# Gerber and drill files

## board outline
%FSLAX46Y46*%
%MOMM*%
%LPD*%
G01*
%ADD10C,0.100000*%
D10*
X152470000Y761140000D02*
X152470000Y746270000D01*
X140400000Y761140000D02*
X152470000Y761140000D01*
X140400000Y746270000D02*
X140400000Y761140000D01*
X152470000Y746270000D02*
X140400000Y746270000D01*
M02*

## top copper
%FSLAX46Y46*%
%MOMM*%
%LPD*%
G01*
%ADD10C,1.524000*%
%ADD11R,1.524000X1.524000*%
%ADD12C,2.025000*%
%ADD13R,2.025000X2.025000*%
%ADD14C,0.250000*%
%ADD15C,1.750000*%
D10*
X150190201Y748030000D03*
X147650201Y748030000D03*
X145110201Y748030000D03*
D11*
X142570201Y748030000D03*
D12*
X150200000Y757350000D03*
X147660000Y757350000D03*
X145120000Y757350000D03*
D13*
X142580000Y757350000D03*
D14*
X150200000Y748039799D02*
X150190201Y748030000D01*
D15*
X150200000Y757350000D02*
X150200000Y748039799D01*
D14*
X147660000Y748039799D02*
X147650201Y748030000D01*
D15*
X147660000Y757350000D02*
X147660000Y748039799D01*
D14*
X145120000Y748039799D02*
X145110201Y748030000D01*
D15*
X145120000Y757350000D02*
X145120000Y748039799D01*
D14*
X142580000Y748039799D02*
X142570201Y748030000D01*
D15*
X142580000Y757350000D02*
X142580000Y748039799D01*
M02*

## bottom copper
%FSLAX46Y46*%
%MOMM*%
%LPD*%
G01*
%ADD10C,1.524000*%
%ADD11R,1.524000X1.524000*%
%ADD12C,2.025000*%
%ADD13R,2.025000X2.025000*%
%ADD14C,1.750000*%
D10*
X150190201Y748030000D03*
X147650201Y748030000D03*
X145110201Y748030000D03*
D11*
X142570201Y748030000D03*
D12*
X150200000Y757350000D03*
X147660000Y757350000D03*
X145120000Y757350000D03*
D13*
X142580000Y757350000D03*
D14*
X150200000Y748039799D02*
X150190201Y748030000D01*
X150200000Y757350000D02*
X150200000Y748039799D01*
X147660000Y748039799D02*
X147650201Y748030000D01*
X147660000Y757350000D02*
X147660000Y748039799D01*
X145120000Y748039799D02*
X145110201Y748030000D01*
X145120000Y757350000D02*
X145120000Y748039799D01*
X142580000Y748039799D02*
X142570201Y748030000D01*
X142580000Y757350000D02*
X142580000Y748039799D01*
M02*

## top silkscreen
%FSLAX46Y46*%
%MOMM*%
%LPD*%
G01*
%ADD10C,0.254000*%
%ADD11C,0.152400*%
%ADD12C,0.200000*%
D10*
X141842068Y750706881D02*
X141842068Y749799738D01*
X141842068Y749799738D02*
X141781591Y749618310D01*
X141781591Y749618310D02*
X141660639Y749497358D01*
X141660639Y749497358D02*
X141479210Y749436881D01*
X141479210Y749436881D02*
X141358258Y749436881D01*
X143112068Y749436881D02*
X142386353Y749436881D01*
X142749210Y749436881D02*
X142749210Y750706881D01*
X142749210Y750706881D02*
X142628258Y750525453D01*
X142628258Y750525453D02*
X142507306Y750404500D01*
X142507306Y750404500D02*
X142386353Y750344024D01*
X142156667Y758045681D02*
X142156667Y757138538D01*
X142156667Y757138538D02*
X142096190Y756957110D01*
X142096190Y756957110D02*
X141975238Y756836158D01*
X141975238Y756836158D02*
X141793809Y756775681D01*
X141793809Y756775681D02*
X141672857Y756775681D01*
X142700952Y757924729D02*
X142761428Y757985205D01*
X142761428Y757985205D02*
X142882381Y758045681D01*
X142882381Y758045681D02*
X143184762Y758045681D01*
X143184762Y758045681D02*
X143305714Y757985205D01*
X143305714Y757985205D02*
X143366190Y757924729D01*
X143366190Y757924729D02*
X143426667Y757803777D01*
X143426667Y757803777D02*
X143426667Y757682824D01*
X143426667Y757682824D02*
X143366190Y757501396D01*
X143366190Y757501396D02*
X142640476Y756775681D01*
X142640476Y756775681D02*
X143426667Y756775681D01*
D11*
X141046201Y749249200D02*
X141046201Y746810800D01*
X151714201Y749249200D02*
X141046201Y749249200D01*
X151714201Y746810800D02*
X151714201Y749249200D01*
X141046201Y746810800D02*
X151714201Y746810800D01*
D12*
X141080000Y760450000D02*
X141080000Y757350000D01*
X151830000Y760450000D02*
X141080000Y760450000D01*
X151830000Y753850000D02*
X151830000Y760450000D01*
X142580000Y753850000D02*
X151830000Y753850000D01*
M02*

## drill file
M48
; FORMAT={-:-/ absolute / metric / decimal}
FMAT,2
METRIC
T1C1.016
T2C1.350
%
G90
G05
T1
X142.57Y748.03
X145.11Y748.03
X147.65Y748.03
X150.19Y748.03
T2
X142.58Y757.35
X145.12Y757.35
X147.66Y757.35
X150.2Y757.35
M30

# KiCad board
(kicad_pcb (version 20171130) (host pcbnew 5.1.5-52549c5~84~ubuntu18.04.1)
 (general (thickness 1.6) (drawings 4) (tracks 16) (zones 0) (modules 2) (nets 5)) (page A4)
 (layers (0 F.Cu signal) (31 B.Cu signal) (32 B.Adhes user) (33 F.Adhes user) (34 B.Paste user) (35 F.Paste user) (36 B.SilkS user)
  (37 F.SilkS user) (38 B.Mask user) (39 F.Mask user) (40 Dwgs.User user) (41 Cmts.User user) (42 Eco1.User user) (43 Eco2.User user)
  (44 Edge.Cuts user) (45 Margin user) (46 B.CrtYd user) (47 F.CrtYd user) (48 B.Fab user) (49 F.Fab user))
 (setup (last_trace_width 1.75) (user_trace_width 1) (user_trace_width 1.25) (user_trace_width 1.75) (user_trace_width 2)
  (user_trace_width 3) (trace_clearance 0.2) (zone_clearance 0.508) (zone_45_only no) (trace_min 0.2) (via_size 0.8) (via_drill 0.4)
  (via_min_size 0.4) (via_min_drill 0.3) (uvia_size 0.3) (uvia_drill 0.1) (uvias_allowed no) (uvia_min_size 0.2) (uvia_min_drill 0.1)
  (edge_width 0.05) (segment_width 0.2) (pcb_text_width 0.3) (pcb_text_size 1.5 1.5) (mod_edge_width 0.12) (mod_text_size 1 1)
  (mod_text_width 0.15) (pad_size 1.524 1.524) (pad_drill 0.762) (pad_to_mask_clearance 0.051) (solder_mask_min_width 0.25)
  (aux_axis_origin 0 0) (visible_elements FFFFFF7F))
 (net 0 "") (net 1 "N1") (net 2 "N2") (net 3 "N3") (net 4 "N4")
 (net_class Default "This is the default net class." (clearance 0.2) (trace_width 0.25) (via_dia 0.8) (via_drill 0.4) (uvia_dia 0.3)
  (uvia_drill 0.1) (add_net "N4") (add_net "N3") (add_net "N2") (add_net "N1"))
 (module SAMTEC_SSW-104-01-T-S (layer F.Cu) (at 150.190201 -748.03)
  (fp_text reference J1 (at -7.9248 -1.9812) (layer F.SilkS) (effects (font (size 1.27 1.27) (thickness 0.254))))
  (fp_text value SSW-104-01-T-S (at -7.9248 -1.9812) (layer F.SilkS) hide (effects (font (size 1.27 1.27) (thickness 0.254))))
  (fp_line (start -9.144 -1.2192) (end -9.144 1.2192) (layer F.SilkS) (width 0.1524))
  (fp_line (start 1.524 -1.2192) (end -9.144 -1.2192) (layer F.SilkS) (width 0.1524))
  (fp_line (start 1.524 1.2192) (end 1.524 -1.2192) (layer F.SilkS) (width 0.1524))
  (fp_line (start -9.144 1.2192) (end 1.524 1.2192) (layer F.SilkS) (width 0.1524))
  (pad 4 thru_hole circle (at 0 0) (size 1.524 1.524) (drill 1.016) (layers *.Cu *.Mask) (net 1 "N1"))
  (pad 3 thru_hole circle (at -2.54 0) (size 1.524 1.524) (drill 1.016) (layers *.Cu *.Mask) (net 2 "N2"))
  (pad 2 thru_hole circle (at -5.08 0) (size 1.524 1.524) (drill 1.016) (layers *.Cu *.Mask) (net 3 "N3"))
  (pad 1 thru_hole rect (at -7.62 0) (size 1.524 1.524) (drill 1.016) (layers *.Cu *.Mask) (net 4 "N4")))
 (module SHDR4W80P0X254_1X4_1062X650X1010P (layer F.Cu) (at 142.58 -757.35)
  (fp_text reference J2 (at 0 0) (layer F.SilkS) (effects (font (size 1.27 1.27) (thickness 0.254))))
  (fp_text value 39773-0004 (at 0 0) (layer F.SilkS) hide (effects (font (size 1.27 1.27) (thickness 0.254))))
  (fp_line (start -1.5 -3.1) (end -1.5 0) (layer F.SilkS) (width 0.2))
  (fp_line (start 9.25 -3.1) (end -1.5 -3.1) (layer F.SilkS) (width 0.2))
  (fp_line (start 9.25 3.5) (end 9.25 -3.1) (layer F.SilkS) (width 0.2))
  (fp_line (start 0 3.5) (end 9.25 3.5) (layer F.SilkS) (width 0.2))
  (pad 4 thru_hole circle (at 7.62 0) (size 2.025 2.025) (drill 1.35) (layers *.Cu *.Mask) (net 1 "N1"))
  (pad 3 thru_hole circle (at 5.08 0) (size 2.025 2.025) (drill 1.35) (layers *.Cu *.Mask) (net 2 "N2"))
  (pad 2 thru_hole circle (at 2.54 0) (size 2.025 2.025) (drill 1.35) (layers *.Cu *.Mask) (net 3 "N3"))
  (pad 1 thru_hole rect (at 0 0) (size 2.025 2.025) (drill 1.35) (layers *.Cu *.Mask) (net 4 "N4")))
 (gr_line (start 152.47 -761.14) (end 152.47 -746.27) (layer Edge.Cuts) (width 0.1))
 (gr_line (start 140.4 -761.14) (end 152.47 -761.14) (layer Edge.Cuts) (width 0.1))
 (gr_line (start 140.4 -746.27) (end 140.4 -761.14) (layer Edge.Cuts) (width 0.1))
 (gr_line (start 152.47 -746.27) (end 140.4 -746.27) (layer Edge.Cuts) (width 0.1))
 (segment (start 150.2 -748.039799) (end 150.190201 -748.03) (width 0.25) (layer F.Cu) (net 1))
 (segment (start 150.2 -757.35) (end 150.2 -748.039799) (width 1.75) (layer F.Cu) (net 1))
 (segment (start 150.2 -748.039799) (end 150.190201 -748.03) (width 1.75) (layer B.Cu) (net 1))
 (segment (start 150.2 -757.35) (end 150.2 -748.039799) (width 1.75) (layer B.Cu) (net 1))
 (segment (start 147.66 -748.039799) (end 147.650201 -748.03) (width 0.25) (layer F.Cu) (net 2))
 (segment (start 147.66 -757.35) (end 147.66 -748.039799) (width 1.75) (layer F.Cu) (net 2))
 (segment (start 147.66 -748.039799) (end 147.650201 -748.03) (width 1.75) (layer B.Cu) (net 2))
 (segment (start 147.66 -757.35) (end 147.66 -748.039799) (width 1.75) (layer B.Cu) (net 2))
 (segment (start 145.12 -748.039799) (end 145.110201 -748.03) (width 0.25) (layer F.Cu) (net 3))
 (segment (start 145.12 -757.35) (end 145.12 -748.039799) (width 1.75) (layer F.Cu) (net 3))
 (segment (start 145.12 -748.039799) (end 145.110201 -748.03) (width 1.75) (layer B.Cu) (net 3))
 (segment (start 145.12 -757.35) (end 145.12 -748.039799) (width 1.75) (layer B.Cu) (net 3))
 (segment (start 142.58 -748.039799) (end 142.570201 -748.03) (width 0.25) (layer F.Cu) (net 4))
 (segment (start 142.58 -757.35) (end 142.58 -748.039799) (width 1.75) (layer F.Cu) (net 4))
 (segment (start 142.58 -748.039799) (end 142.570201 -748.03) (width 1.75) (layer B.Cu) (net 4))
 (segment (start 142.58 -757.35) (end 142.58 -748.039799) (width 1.75) (layer B.Cu) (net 4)))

